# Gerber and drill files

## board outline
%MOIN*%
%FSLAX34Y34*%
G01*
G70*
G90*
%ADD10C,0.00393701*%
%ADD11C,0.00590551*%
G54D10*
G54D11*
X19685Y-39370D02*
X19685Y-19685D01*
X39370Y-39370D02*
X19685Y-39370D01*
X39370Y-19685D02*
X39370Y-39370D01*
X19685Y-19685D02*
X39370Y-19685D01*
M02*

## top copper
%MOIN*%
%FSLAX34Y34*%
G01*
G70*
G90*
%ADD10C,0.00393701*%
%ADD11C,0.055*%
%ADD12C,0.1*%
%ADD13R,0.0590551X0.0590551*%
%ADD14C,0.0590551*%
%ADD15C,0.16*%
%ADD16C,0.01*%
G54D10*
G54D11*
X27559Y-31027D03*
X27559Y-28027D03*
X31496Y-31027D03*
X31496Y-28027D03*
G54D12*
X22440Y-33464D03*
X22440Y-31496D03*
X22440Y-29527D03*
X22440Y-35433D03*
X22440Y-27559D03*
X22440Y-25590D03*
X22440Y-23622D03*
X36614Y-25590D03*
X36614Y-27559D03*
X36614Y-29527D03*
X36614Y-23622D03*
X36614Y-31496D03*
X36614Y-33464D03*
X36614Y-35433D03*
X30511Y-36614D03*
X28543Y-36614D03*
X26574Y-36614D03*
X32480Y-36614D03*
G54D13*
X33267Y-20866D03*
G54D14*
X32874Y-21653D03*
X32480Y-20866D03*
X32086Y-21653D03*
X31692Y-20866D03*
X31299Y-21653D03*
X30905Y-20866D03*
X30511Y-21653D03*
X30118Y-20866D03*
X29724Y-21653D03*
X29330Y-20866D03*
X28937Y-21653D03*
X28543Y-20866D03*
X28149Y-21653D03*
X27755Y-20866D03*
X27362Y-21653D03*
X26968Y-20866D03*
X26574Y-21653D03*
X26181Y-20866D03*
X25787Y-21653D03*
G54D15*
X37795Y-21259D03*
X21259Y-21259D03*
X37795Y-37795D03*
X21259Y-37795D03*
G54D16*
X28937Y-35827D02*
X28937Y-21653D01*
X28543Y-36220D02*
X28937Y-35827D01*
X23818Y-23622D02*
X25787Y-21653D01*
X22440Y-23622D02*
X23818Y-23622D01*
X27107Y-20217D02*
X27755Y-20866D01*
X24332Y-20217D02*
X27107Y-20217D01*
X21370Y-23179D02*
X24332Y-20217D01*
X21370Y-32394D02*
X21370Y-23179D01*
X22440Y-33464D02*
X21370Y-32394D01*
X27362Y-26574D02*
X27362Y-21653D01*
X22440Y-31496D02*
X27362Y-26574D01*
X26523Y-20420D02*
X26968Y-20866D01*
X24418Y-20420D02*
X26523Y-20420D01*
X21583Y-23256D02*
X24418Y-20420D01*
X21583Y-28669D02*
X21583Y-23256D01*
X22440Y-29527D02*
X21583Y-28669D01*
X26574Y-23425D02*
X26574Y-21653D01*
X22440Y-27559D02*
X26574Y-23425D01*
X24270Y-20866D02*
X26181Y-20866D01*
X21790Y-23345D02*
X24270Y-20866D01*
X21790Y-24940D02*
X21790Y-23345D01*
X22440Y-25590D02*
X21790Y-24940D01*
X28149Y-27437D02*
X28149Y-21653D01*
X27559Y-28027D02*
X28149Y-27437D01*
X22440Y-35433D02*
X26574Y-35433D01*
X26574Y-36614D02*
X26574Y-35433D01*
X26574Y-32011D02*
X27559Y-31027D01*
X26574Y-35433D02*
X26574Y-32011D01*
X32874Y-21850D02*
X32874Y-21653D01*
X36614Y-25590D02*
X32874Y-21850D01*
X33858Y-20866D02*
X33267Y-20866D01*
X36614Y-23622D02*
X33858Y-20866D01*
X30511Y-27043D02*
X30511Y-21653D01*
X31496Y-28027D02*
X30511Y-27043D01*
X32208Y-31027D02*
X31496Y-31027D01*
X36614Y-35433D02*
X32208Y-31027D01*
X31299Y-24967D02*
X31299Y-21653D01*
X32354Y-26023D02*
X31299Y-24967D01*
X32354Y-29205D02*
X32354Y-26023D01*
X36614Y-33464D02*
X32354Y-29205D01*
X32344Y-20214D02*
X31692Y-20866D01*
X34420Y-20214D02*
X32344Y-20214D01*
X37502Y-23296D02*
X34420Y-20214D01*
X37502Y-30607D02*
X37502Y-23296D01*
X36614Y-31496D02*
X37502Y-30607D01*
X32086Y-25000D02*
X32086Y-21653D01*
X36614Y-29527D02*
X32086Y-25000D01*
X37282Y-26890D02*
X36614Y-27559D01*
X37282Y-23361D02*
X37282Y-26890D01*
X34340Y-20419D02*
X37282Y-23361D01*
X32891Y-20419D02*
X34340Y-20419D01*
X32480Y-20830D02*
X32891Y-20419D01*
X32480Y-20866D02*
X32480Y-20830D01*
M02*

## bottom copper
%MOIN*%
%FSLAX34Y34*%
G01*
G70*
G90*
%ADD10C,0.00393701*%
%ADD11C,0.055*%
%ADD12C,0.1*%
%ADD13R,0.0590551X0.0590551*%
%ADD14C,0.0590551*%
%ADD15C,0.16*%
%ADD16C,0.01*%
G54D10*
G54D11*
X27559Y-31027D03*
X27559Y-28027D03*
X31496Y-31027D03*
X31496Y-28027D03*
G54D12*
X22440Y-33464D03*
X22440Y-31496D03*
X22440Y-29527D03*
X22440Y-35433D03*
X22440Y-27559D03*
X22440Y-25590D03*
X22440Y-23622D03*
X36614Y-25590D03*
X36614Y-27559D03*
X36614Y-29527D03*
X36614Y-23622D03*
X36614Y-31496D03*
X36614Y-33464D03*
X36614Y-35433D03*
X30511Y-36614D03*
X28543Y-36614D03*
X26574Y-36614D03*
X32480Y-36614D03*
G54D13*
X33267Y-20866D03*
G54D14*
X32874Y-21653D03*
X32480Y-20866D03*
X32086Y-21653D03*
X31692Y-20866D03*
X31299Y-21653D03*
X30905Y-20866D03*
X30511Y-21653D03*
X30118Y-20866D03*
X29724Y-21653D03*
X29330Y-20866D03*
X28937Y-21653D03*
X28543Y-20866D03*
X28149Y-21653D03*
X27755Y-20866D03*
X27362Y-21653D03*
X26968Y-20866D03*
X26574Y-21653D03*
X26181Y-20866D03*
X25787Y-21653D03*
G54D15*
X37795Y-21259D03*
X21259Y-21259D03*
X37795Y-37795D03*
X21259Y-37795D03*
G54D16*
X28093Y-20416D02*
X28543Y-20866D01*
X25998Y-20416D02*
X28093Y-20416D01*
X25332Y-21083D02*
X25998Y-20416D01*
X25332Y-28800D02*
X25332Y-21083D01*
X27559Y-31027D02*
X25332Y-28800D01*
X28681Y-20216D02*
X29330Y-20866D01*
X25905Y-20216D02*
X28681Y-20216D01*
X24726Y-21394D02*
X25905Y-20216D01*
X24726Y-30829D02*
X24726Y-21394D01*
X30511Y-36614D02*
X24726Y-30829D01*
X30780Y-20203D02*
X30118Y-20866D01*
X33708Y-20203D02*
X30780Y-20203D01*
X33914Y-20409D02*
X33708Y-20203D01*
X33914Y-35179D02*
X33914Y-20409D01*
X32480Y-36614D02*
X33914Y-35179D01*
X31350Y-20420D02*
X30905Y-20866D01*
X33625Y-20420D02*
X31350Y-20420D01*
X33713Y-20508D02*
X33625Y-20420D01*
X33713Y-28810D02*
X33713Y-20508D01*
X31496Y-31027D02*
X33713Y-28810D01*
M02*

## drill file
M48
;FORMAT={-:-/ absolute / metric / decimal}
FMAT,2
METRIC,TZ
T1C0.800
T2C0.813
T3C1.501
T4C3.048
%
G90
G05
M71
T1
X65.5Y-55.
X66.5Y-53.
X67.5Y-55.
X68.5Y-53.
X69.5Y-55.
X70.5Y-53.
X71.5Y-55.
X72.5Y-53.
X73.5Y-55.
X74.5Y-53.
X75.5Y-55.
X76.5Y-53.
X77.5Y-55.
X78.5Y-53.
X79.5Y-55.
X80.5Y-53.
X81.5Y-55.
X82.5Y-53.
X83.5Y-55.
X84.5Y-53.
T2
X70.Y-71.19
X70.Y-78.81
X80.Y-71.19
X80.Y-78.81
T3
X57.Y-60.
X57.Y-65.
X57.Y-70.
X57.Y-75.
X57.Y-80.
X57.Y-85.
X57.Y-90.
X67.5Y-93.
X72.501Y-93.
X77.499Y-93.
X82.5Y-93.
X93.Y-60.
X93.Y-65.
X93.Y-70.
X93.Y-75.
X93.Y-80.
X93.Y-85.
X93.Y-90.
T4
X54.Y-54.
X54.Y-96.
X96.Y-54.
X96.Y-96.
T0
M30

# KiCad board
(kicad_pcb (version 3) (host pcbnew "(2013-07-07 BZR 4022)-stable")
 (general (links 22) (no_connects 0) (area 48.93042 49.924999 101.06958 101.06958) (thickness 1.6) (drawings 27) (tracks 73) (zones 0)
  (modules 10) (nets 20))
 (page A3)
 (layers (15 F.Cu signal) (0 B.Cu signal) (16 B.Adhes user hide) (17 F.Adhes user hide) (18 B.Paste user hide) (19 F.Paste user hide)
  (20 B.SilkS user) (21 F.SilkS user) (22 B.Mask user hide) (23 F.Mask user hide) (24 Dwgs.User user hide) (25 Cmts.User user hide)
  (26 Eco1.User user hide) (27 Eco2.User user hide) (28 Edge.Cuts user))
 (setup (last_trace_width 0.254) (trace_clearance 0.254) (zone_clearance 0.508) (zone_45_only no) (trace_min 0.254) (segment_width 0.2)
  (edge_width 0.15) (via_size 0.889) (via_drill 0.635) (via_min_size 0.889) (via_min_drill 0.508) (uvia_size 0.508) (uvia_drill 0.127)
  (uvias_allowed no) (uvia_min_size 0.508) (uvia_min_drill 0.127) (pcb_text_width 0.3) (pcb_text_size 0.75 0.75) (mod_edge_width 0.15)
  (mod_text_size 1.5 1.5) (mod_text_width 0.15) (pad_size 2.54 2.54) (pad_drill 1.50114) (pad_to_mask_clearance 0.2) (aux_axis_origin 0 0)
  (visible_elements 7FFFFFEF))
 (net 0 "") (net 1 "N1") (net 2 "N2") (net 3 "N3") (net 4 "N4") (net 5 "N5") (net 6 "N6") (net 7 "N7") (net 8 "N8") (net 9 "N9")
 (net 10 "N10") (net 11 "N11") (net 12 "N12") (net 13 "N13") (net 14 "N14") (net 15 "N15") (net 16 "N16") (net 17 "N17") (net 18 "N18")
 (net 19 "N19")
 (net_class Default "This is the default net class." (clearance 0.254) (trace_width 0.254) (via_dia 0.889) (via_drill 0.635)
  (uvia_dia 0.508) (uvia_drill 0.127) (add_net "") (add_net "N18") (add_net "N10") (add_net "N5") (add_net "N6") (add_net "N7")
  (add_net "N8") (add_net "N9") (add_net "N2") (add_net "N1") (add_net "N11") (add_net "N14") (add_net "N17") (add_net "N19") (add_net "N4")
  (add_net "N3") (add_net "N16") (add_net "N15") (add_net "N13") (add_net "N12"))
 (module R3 (layer F.Cu) (at 70 75 90) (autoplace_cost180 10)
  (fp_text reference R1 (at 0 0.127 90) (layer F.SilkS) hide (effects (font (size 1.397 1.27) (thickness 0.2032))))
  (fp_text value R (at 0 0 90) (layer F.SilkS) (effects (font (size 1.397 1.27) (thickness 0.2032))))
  (pad 1 thru_hole circle (at -3.81 0 90) (size 1.397 1.397) (drill 0.8128) (layers *.Cu *.Mask F.SilkS) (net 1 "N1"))
  (pad 2 thru_hole circle (at 3.81 0 90) (size 1.397 1.397) (drill 0.8128) (layers *.Cu *.Mask F.SilkS) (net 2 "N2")))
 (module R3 (layer F.Cu) (at 80 75 90) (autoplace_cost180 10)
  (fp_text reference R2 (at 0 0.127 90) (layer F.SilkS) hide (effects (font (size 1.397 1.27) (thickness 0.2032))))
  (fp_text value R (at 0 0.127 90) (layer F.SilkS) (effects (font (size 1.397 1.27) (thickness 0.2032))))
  (pad 1 thru_hole circle (at -3.81 0 90) (size 1.397 1.397) (drill 0.8128) (layers *.Cu *.Mask F.SilkS) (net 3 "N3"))
  (pad 2 thru_hole circle (at 3.81 0 90) (size 1.397 1.397) (drill 0.8128) (layers *.Cu *.Mask F.SilkS) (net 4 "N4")))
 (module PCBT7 (layer F.Cu) (at 57 75 90)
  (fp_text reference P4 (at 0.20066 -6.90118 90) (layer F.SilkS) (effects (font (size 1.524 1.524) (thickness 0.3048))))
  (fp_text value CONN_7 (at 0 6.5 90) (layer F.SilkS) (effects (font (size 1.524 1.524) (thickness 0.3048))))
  (pad 6 thru_hole circle (at -10 0 90) (size 2.54 2.54) (drill 1.50114) (layers *.Cu *.Mask F.SilkS) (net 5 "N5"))
  (pad 5 thru_hole circle (at -5 0 90) (size 2.54 2.54) (drill 1.50114) (layers *.Cu *.Mask F.SilkS) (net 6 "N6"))
  (pad 4 thru_hole circle (at 0 0 90) (size 2.54 2.54) (drill 1.50114) (layers *.Cu *.Mask F.SilkS) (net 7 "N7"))
  (pad 7 thru_hole circle (at -15 0 90) (size 2.54 2.54) (drill 1.50114) (layers *.Cu *.Mask F.SilkS) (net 1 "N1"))
  (pad 3 thru_hole circle (at 5 0 90) (size 2.54 2.54) (drill 1.50114) (layers *.Cu *.Mask F.SilkS) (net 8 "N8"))
  (pad 2 thru_hole circle (at 10 0 90) (size 2.54 2.54) (drill 1.50114) (layers *.Cu *.Mask F.SilkS) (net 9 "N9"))
  (pad 1 thru_hole circle (at 15 0 90) (size 2.54 2.54) (drill 1.50114) (layers *.Cu *.Mask F.SilkS) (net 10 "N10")))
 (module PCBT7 (layer F.Cu) (at 93 75 270)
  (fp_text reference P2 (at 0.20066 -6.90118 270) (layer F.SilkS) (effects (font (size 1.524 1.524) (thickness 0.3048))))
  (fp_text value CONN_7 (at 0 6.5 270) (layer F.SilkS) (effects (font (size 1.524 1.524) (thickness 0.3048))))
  (pad 2 thru_hole circle (at -10 0 270) (size 2.54 2.54) (drill 1.50114) (layers *.Cu *.Mask F.SilkS) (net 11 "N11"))
  (pad 3 thru_hole circle (at -5 0 270) (size 2.54 2.54) (drill 1.50114) (layers *.Cu *.Mask F.SilkS) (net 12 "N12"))
  (pad 4 thru_hole circle (at 0 0 270) (size 2.54 2.54) (drill 1.50114) (layers *.Cu *.Mask F.SilkS) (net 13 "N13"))
  (pad 1 thru_hole circle (at -15 0 270) (size 2.54 2.54) (drill 1.50114) (layers *.Cu *.Mask F.SilkS) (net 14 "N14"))
  (pad 5 thru_hole circle (at 5 0 270) (size 2.54 2.54) (drill 1.50114) (layers *.Cu *.Mask F.SilkS) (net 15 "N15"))
  (pad 6 thru_hole circle (at 10 0 270) (size 2.54 2.54) (drill 1.50114) (layers *.Cu *.Mask F.SilkS) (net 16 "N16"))
  (pad 7 thru_hole circle (at 15 0 270) (size 2.54 2.54) (drill 1.50114) (layers *.Cu *.Mask F.SilkS) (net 3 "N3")))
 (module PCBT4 (layer F.Cu) (at 75 93 180)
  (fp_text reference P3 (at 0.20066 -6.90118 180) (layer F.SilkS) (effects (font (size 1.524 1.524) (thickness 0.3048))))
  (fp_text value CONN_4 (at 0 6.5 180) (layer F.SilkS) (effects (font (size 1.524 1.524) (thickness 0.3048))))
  (pad 2 thru_hole circle (at -2.49936 0 180) (size 2.54 2.54) (drill 1.50114) (layers *.Cu *.Mask F.SilkS) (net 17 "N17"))
  (pad 3 thru_hole circle (at 2.49936 0 180) (size 2.54 2.54) (drill 1.50114) (layers *.Cu *.Mask F.SilkS) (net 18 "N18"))
  (pad 4 thru_hole circle (at 7.5 0 180) (size 2.54 2.54) (drill 1.50114) (layers *.Cu *.Mask F.SilkS) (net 1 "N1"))
  (pad 1 thru_hole circle (at -7.5 0 180) (size 2.54 2.54) (drill 1.50114) (layers *.Cu *.Mask F.SilkS) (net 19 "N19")))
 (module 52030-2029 (layer F.Cu) (at 84.5 55 180)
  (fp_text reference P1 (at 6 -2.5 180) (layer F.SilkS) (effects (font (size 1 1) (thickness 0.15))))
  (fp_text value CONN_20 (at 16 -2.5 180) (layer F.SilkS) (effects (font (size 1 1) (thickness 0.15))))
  (pad 1 thru_hole rect (at 0 2 180) (size 1.5 1.5) (drill 0.8) (layers *.Cu *.Mask F.SilkS) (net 14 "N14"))
  (pad 2 thru_hole circle (at 1 0 180) (size 1.5 1.5) (drill 0.8) (layers *.Cu *.Mask F.SilkS) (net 11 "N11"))
  (pad 3 thru_hole circle (at 2 2 180) (size 1.5 1.5) (drill 0.8) (layers *.Cu *.Mask F.SilkS) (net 12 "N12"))
  (pad 4 thru_hole circle (at 3 0 180) (size 1.5 1.5) (drill 0.8) (layers *.Cu *.Mask F.SilkS) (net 13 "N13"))
  (pad 5 thru_hole circle (at 4 2 180) (size 1.5 1.5) (drill 0.8) (layers *.Cu *.Mask F.SilkS) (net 15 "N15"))
  (pad 6 thru_hole circle (at 5 0 180) (size 1.5 1.5) (drill 0.8) (layers *.Cu *.Mask F.SilkS) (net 16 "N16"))
  (pad 7 thru_hole circle (at 6 2 180) (size 1.5 1.5) (drill 0.8) (layers *.Cu *.Mask F.SilkS) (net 3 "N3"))
  (pad 8 thru_hole circle (at 7 0 180) (size 1.5 1.5) (drill 0.8) (layers *.Cu *.Mask F.SilkS) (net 4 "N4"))
  (pad 9 thru_hole circle (at 8 2 180) (size 1.5 1.5) (drill 0.8) (layers *.Cu *.Mask F.SilkS) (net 19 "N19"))
  (pad 10 thru_hole circle (at 9 0 180) (size 1.5 1.5) (drill 0.8) (layers *.Cu *.Mask F.SilkS))
  (pad 11 thru_hole circle (at 10 2 180) (size 1.5 1.5) (drill 0.8) (layers *.Cu *.Mask F.SilkS) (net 17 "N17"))
  (pad 12 thru_hole circle (at 11 0 180) (size 1.5 1.5) (drill 0.8) (layers *.Cu *.Mask F.SilkS) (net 18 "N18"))
  (pad 13 thru_hole circle (at 12 2 180) (size 1.5 1.5) (drill 0.8) (layers *.Cu *.Mask F.SilkS) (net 1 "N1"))
  (pad 14 thru_hole circle (at 13 0 180) (size 1.5 1.5) (drill 0.8) (layers *.Cu *.Mask F.SilkS) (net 2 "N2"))
  (pad 15 thru_hole circle (at 14 2 180) (size 1.5 1.5) (drill 0.8) (layers *.Cu *.Mask F.SilkS) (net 5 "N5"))
  (pad 16 thru_hole circle (at 15 0 180) (size 1.5 1.5) (drill 0.8) (layers *.Cu *.Mask F.SilkS) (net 6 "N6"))
  (pad 17 thru_hole circle (at 16 2 180) (size 1.5 1.5) (drill 0.8) (layers *.Cu *.Mask F.SilkS) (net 7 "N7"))
  (pad 18 thru_hole circle (at 17 0 180) (size 1.5 1.5) (drill 0.8) (layers *.Cu *.Mask F.SilkS) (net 8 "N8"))
  (pad 19 thru_hole circle (at 18 2 180) (size 1.5 1.5) (drill 0.8) (layers *.Cu *.Mask F.SilkS) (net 9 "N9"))
  (pad 20 thru_hole circle (at 19 0 180) (size 1.5 1.5) (drill 0.8) (layers *.Cu *.Mask F.SilkS) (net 10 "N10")))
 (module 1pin (layer F.Cu) (at 96 54)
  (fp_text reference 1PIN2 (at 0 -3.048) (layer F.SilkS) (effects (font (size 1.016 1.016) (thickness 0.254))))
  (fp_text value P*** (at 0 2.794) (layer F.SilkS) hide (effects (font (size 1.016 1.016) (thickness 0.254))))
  (pad 1 thru_hole circle (at 0 0) (size 4.064 4.064) (drill 3.048) (layers *.Cu *.Mask F.SilkS)))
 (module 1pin (layer F.Cu) (at 54 54)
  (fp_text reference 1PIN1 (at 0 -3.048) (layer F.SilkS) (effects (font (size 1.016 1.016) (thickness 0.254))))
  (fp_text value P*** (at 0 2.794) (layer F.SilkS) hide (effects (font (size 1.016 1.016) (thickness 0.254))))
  (pad 1 thru_hole circle (at 0 0) (size 4.064 4.064) (drill 3.048) (layers *.Cu *.Mask F.SilkS)))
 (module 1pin (layer F.Cu) (at 96 96)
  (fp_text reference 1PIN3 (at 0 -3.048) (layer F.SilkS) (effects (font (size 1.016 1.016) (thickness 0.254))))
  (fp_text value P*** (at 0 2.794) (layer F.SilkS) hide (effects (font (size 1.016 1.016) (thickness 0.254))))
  (pad 1 thru_hole circle (at 0 0) (size 4.064 4.064) (drill 3.048) (layers *.Cu *.Mask F.SilkS)))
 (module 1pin (layer F.Cu) (at 54 96)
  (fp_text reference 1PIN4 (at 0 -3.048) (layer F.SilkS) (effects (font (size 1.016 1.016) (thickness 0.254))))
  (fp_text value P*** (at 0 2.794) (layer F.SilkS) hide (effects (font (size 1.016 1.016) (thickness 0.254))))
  (pad 1 thru_hole circle (at 0 0) (size 4.064 4.064) (drill 3.048) (layers *.Cu *.Mask F.SilkS)))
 (gr_line (start 50 100) (end 50 50) (angle 90) (layer Edge.Cuts) (width 0.15))
 (gr_line (start 100 100) (end 50 100) (angle 90) (layer Edge.Cuts) (width 0.15))
 (gr_line (start 100 50) (end 100 100) (angle 90) (layer Edge.Cuts) (width 0.15))
 (gr_line (start 50 50) (end 100 50) (angle 90) (layer Edge.Cuts) (width 0.15))
 (segment (start 73.5 91.0006) (end 73.5 55) (width 0.254) (layer F.Cu) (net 18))
 (segment (start 72.5006 92) (end 73.5 91.0006) (width 0.254) (layer F.Cu) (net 18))
 (segment (start 60.5 60) (end 65.5 55) (width 0.254) (layer F.Cu) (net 10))
 (segment (start 57 60) (end 60.5 60) (width 0.254) (layer F.Cu) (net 10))
 (segment (start 68.8531 51.3531) (end 70.5 53) (width 0.254) (layer F.Cu) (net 5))
 (segment (start 61.8047 51.3531) (end 68.8531 51.3531) (width 0.254) (layer F.Cu) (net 5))
 (segment (start 54.2822 58.8756) (end 61.8047 51.3531) (width 0.254) (layer F.Cu) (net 5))
 (segment (start 54.2822 82.2822) (end 54.2822 58.8756) (width 0.254) (layer F.Cu) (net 5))
 (segment (start 57 85) (end 54.2822 82.2822) (width 0.254) (layer F.Cu) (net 5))
 (segment (start 69.5 67.5) (end 69.5 55) (width 0.254) (layer F.Cu) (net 6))
 (segment (start 57 80) (end 69.5 67.5) (width 0.254) (layer F.Cu) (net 6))
 (segment (start 67.3687 51.8687) (end 68.5 53) (width 0.254) (layer F.Cu) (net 7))
 (segment (start 62.0241 51.8687) (end 67.3687 51.8687) (width 0.254) (layer F.Cu) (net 7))
 (segment (start 54.8211 59.0717) (end 62.0241 51.8687) (width 0.254) (layer F.Cu) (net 7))
 (segment (start 54.8211 72.8211) (end 54.8211 59.0717) (width 0.254) (layer F.Cu) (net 7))
 (segment (start 57 75) (end 54.8211 72.8211) (width 0.254) (layer F.Cu) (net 7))
 (segment (start 67.5 59.5) (end 67.5 55) (width 0.254) (layer F.Cu) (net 8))
 (segment (start 57 70) (end 67.5 59.5) (width 0.254) (layer F.Cu) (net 8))
 (segment (start 61.6466 53) (end 66.5 53) (width 0.254) (layer F.Cu) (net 9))
 (segment (start 55.3485 59.2981) (end 61.6466 53) (width 0.254) (layer F.Cu) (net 9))
 (segment (start 55.3485 63.3485) (end 55.3485 59.2981) (width 0.254) (layer F.Cu) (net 9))
 (segment (start 57 65) (end 55.3485 63.3485) (width 0.254) (layer F.Cu) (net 9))
 (segment (start 71.5 69.69) (end 71.5 55) (width 0.254) (layer F.Cu) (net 2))
 (segment (start 70 71.19) (end 71.5 69.69) (width 0.254) (layer F.Cu) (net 2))
 (segment (start 71.3581 51.8581) (end 72.5 53) (width 0.254) (layer B.Cu) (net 1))
 (segment (start 66.0368 51.8581) (end 71.3581 51.8581) (width 0.254) (layer B.Cu) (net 1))
 (segment (start 64.3437 53.5512) (end 66.0368 51.8581) (width 0.254) (layer B.Cu) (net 1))
 (segment (start 64.3437 73.1537) (end 64.3437 53.5512) (width 0.254) (layer B.Cu) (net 1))
 (segment (start 70 78.81) (end 64.3437 73.1537) (width 0.254) (layer B.Cu) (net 1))
 (segment (start 57 90) (end 67.5 90) (width 0.254) (layer F.Cu) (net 1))
 (segment (start 67.5 93) (end 67.5 90) (width 0.254) (layer F.Cu) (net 1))
 (segment (start 67.5 81.31) (end 70 78.81) (width 0.254) (layer F.Cu) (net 1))
 (segment (start 67.5 90) (end 67.5 81.31) (width 0.254) (layer F.Cu) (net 1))
 (segment (start 83.5 55.5) (end 83.5 55) (width 0.254) (layer F.Cu) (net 11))
 (segment (start 93 65) (end 83.5 55.5) (width 0.254) (layer F.Cu) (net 11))
 (segment (start 86 53) (end 84.5 53) (width 0.254) (layer F.Cu) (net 14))
 (segment (start 93 60) (end 86 53) (width 0.254) (layer F.Cu) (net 14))
 (segment (start 72.8498 51.3498) (end 74.5 53) (width 0.254) (layer B.Cu) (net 17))
 (segment (start 65.7987 51.3498) (end 72.8498 51.3498) (width 0.254) (layer B.Cu) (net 17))
 (segment (start 62.8057 54.3428) (end 65.7987 51.3498) (width 0.254) (layer B.Cu) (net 17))
 (segment (start 62.8057 78.3063) (end 62.8057 54.3428) (width 0.254) (layer B.Cu) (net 17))
 (segment (start 77.4994 93) (end 62.8057 78.3063) (width 0.254) (layer B.Cu) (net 17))
 (segment (start 78.1834 51.3166) (end 76.5 53) (width 0.254) (layer B.Cu) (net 19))
 (segment (start 85.6193 51.3166) (end 78.1834 51.3166) (width 0.254) (layer B.Cu) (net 19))
 (segment (start 86.143 51.8403) (end 85.6193 51.3166) (width 0.254) (layer B.Cu) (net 19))
 (segment (start 86.143 89.357) (end 86.143 51.8403) (width 0.254) (layer B.Cu) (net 19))
 (segment (start 82.5 93) (end 86.143 89.357) (width 0.254) (layer B.Cu) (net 19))
 (segment (start 77.5 68.69) (end 77.5 55) (width 0.254) (layer F.Cu) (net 4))
 (segment (start 80 71.19) (end 77.5 68.69) (width 0.254) (layer F.Cu) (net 4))
 (segment (start 81.81 78.81) (end 80 78.81) (width 0.254) (layer F.Cu) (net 3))
 (segment (start 93 90) (end 81.81 78.81) (width 0.254) (layer F.Cu) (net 3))
 (segment (start 79.6313 51.8687) (end 78.5 53) (width 0.254) (layer B.Cu) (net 3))
 (segment (start 85.4079 51.8687) (end 79.6313 51.8687) (width 0.254) (layer B.Cu) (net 3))
 (segment (start 85.6313 52.0921) (end 85.4079 51.8687) (width 0.254) (layer B.Cu) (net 3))
 (segment (start 85.6313 73.1787) (end 85.6313 52.0921) (width 0.254) (layer B.Cu) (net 3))
 (segment (start 80 78.81) (end 85.6313 73.1787) (width 0.254) (layer B.Cu) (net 3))
 (segment (start 79.5 63.4178) (end 79.5 55) (width 0.254) (layer F.Cu) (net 16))
 (segment (start 82.1808 66.0986) (end 79.5 63.4178) (width 0.254) (layer F.Cu) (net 16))
 (segment (start 82.1808 74.1808) (end 82.1808 66.0986) (width 0.254) (layer F.Cu) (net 16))
 (segment (start 93 85) (end 82.1808 74.1808) (width 0.254) (layer F.Cu) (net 16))
 (segment (start 82.1555 51.3445) (end 80.5 53) (width 0.254) (layer F.Cu) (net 15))
 (segment (start 87.4287 51.3445) (end 82.1555 51.3445) (width 0.254) (layer F.Cu) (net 15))
 (segment (start 95.2566 59.1724) (end 87.4287 51.3445) (width 0.254) (layer F.Cu) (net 15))
 (segment (start 95.2566 77.7434) (end 95.2566 59.1724) (width 0.254) (layer F.Cu) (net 15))
 (segment (start 93 80) (end 95.2566 77.7434) (width 0.254) (layer F.Cu) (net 15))
 (segment (start 81.5 63.5) (end 81.5 55) (width 0.254) (layer F.Cu) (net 13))
 (segment (start 93 75) (end 81.5 63.5) (width 0.254) (layer F.Cu) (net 13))
 (segment (start 94.6972 68.3028) (end 93 70) (width 0.254) (layer F.Cu) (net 12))
 (segment (start 94.6972 59.3382) (end 94.6972 68.3028) (width 0.254) (layer F.Cu) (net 12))
 (segment (start 87.2238 51.8648) (end 94.6972 59.3382) (width 0.254) (layer F.Cu) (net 12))
 (segment (start 83.5441 51.8648) (end 87.2238 51.8648) (width 0.254) (layer F.Cu) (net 12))
 (segment (start 82.5 52.9089) (end 83.5441 51.8648) (width 0.254) (layer F.Cu) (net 12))
 (segment (start 82.5 53) (end 82.5 52.9089) (width 0.254) (layer F.Cu) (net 12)))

